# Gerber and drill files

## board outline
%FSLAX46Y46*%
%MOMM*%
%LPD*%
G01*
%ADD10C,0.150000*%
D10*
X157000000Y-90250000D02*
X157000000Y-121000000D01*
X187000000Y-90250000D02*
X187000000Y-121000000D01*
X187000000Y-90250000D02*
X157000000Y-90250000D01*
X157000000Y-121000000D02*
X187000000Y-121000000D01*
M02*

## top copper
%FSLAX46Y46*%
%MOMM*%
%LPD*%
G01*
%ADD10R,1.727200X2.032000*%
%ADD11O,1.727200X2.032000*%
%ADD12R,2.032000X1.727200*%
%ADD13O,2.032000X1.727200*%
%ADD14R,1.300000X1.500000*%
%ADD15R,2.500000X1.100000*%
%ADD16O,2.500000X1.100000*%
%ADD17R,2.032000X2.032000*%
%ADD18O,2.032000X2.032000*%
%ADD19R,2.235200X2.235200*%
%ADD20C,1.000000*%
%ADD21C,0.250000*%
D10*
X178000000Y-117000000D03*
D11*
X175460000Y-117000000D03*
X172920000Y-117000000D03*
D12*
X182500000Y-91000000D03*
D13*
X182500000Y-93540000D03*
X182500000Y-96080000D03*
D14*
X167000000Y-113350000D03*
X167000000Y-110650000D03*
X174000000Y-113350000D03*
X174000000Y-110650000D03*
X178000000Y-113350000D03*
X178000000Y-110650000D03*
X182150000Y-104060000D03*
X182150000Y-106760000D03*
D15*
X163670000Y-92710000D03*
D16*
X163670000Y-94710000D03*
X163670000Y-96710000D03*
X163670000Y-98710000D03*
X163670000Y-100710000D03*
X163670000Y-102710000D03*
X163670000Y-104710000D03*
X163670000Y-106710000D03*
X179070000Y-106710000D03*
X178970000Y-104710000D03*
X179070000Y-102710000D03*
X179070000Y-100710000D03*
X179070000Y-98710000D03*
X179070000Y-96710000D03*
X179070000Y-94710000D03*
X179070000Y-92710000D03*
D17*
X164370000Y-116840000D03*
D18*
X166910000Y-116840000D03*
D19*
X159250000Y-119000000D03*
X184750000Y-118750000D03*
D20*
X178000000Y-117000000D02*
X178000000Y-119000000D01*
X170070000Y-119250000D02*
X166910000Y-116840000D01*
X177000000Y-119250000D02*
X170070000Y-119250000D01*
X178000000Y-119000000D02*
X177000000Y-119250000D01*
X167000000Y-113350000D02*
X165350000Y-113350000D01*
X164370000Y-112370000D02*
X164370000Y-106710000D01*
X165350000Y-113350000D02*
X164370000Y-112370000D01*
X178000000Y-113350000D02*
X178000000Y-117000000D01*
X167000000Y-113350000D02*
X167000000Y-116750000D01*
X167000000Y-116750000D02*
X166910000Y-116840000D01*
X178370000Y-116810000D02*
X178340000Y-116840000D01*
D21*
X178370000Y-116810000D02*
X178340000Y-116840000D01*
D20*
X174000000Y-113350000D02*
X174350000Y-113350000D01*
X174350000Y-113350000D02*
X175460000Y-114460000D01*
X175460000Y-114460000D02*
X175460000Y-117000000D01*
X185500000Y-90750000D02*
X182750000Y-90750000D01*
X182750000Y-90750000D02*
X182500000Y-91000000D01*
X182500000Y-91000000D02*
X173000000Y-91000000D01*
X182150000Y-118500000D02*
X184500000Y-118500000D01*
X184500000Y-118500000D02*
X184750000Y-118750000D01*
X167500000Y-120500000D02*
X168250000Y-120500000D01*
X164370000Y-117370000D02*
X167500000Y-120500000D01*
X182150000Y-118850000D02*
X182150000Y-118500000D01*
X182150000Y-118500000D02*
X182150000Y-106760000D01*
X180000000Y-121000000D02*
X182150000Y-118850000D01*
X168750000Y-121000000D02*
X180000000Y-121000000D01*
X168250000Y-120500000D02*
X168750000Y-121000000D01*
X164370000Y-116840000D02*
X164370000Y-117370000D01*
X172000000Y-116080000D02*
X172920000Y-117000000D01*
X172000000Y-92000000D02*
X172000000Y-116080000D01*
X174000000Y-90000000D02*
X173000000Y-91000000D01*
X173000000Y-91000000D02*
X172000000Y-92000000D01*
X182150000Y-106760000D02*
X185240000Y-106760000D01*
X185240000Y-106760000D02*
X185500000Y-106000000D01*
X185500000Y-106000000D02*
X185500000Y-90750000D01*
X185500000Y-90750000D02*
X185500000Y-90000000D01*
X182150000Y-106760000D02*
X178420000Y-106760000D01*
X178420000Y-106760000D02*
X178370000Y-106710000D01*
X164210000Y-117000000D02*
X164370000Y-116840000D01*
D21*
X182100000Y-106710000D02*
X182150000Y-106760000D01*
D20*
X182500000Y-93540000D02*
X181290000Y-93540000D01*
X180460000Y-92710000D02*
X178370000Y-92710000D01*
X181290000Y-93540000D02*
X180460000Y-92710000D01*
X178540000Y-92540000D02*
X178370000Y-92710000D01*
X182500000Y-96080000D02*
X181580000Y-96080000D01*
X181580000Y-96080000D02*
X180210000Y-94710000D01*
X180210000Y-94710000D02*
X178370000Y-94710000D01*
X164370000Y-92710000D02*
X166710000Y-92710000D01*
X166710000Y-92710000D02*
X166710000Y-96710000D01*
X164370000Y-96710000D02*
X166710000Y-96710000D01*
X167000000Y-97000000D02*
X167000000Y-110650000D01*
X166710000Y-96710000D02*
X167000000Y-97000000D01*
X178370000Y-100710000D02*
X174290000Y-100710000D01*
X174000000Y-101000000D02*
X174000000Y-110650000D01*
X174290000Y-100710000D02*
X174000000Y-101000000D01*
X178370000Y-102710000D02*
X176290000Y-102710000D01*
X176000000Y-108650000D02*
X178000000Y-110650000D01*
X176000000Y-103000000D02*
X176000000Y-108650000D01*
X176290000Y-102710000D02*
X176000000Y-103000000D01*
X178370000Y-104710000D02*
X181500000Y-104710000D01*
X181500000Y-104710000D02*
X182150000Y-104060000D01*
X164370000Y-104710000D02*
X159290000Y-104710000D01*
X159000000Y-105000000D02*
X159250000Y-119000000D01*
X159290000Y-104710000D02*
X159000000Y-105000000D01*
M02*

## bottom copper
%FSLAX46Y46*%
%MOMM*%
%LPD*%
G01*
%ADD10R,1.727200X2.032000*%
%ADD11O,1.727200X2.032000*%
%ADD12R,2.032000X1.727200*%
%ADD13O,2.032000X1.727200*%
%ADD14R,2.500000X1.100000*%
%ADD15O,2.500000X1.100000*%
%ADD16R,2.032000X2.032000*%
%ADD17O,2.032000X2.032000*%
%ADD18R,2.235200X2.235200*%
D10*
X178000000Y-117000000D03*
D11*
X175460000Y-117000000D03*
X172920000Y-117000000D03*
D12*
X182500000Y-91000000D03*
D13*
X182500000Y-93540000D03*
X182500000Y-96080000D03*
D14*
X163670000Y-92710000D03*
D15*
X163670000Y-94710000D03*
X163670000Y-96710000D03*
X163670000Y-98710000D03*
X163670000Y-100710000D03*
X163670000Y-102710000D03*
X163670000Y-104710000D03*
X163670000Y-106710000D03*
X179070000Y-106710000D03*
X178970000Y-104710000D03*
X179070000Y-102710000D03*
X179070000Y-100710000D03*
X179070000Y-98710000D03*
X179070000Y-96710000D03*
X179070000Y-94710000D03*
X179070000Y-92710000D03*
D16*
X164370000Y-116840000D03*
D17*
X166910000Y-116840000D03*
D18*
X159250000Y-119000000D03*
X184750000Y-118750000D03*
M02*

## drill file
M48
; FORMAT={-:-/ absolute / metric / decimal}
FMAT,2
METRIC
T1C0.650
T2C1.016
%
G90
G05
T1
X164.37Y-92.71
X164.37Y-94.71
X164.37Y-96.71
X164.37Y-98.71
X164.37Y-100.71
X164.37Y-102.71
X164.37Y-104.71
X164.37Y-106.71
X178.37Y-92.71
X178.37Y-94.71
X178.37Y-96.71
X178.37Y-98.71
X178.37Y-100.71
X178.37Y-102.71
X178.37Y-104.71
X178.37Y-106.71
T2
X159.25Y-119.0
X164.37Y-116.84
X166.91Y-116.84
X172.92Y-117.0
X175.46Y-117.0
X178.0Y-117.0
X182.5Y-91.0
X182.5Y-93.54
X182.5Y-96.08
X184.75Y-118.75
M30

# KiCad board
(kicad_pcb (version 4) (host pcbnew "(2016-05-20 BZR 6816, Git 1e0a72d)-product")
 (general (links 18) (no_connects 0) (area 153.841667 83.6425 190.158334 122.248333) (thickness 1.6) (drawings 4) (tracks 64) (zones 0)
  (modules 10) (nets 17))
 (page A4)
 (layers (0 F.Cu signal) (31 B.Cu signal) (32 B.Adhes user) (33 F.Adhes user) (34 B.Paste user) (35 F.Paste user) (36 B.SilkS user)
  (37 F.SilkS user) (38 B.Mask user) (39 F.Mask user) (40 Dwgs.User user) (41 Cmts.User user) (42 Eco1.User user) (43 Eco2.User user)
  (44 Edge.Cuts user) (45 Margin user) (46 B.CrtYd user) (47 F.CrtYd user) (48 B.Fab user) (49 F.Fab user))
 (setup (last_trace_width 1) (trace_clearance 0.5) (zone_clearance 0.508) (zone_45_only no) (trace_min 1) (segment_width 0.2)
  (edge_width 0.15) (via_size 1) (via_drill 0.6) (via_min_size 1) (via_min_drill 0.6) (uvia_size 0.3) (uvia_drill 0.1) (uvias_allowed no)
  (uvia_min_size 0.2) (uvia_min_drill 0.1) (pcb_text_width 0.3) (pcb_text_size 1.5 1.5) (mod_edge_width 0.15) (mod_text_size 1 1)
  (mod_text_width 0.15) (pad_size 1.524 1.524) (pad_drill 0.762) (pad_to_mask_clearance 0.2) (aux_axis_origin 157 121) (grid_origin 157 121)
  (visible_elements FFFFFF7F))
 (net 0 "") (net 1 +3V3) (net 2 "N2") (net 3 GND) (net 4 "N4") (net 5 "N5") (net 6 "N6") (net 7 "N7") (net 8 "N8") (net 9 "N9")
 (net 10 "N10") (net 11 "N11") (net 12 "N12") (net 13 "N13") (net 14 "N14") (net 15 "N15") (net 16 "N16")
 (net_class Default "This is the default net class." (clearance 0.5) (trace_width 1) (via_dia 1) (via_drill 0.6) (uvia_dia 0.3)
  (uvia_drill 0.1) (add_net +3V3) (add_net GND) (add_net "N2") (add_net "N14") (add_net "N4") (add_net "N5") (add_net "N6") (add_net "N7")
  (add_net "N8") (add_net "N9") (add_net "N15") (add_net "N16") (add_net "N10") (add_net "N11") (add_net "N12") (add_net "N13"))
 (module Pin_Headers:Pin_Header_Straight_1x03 (layer F.Cu) (at 178 117 270)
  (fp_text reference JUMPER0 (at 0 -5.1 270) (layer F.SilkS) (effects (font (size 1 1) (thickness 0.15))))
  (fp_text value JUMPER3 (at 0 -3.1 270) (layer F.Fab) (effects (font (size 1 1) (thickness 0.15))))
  (pad 1 thru_hole rect (at 0 0 270) (size 2.032 1.7272) (drill 1.016) (layers *.Cu *.Mask F.SilkS) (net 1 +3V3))
  (pad 2 thru_hole oval (at 0 2.54 270) (size 2.032 1.7272) (drill 1.016) (layers *.Cu *.Mask F.SilkS) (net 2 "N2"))
  (pad 3 thru_hole oval (at 0 5.08 270) (size 2.032 1.7272) (drill 1.016) (layers *.Cu *.Mask F.SilkS) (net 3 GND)))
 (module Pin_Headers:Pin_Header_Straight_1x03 (layer F.Cu) (at 182.5 91)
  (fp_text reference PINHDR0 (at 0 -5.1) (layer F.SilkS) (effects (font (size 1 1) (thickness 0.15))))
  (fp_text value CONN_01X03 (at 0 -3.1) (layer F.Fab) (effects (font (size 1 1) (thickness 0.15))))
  (pad 1 thru_hole rect (at 0 0) (size 2.032 1.7272) (drill 1.016) (layers *.Cu *.Mask F.SilkS) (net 3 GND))
  (pad 2 thru_hole oval (at 0 2.54) (size 2.032 1.7272) (drill 1.016) (layers *.Cu *.Mask F.SilkS) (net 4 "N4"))
  (pad 3 thru_hole oval (at 0 5.08) (size 2.032 1.7272) (drill 1.016) (layers *.Cu *.Mask F.SilkS) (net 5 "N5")))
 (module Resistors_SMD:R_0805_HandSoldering (layer F.Cu) (at 167 112 90)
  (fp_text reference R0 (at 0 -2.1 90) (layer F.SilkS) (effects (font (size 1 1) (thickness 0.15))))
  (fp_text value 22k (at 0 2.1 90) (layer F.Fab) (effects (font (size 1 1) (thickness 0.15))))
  (pad 1 smd rect (at -1.35 0 90) (size 1.5 1.3) (layers F.Cu F.Paste F.Mask) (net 1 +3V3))
  (pad 2 smd rect (at 1.35 0 90) (size 1.5 1.3) (layers F.Cu F.Paste F.Mask) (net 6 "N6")))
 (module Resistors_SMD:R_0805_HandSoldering (layer F.Cu) (at 174 112 90)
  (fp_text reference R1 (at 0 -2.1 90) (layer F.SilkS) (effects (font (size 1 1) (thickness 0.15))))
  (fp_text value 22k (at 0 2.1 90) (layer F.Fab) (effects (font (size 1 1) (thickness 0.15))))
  (pad 1 smd rect (at -1.35 0 90) (size 1.5 1.3) (layers F.Cu F.Paste F.Mask) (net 2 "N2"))
  (pad 2 smd rect (at 1.35 0 90) (size 1.5 1.3) (layers F.Cu F.Paste F.Mask) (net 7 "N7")))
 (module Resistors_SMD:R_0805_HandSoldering (layer F.Cu) (at 178 112 90)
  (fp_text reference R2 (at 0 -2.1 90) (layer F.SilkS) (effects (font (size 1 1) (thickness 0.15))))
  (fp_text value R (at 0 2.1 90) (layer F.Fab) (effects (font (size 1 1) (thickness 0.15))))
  (pad 1 smd rect (at -1.35 0 90) (size 1.5 1.3) (layers F.Cu F.Paste F.Mask) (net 1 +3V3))
  (pad 2 smd rect (at 1.35 0 90) (size 1.5 1.3) (layers F.Cu F.Paste F.Mask) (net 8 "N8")))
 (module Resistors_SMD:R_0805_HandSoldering (layer F.Cu) (at 182.15 105.41 270)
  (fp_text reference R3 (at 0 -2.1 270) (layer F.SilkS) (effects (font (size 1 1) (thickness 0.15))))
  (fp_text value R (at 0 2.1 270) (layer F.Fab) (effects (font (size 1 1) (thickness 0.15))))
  (pad 1 smd rect (at -1.35 0 270) (size 1.5 1.3) (layers F.Cu F.Paste F.Mask) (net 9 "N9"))
  (pad 2 smd rect (at 1.35 0 270) (size 1.5 1.3) (layers F.Cu F.Paste F.Mask) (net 3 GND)))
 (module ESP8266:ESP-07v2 (layer F.Cu) (at 164.37 92.71)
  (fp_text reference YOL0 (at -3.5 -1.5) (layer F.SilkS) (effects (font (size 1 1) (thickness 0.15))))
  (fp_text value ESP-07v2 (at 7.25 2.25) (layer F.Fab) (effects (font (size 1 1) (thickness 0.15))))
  (pad 1 thru_hole rect (at 0 0) (size 2.5 1.1) (drill 0.65 (offset -0.7 0)) (layers *.Cu *.Mask F.SilkS) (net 6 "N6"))
  (pad 2 thru_hole oval (at 0 2) (size 2.5 1.1) (drill 0.65 (offset -0.7 0)) (layers *.Cu *.Mask F.SilkS) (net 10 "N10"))
  (pad 3 thru_hole oval (at 0 4) (size 2.5 1.1) (drill 0.65 (offset -0.7 0)) (layers *.Cu *.Mask F.SilkS) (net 6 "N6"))
  (pad 4 thru_hole oval (at 0 6) (size 2.5 1.1) (drill 0.65 (offset -0.7 0)) (layers *.Cu *.Mask F.SilkS) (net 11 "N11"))
  (pad 5 thru_hole oval (at 0 8) (size 2.5 1.1) (drill 0.65 (offset -0.7 0)) (layers *.Cu *.Mask F.SilkS) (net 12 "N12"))
  (pad 6 thru_hole oval (at 0 10) (size 2.5 1.1) (drill 0.65 (offset -0.7 0)) (layers *.Cu *.Mask F.SilkS) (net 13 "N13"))
  (pad 7 thru_hole oval (at 0 12) (size 2.5 1.1) (drill 0.65 (offset -0.7 0)) (layers *.Cu *.Mask F.SilkS) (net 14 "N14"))
  (pad 8 thru_hole oval (at 0 14) (size 2.5 1.1) (drill 0.65 (offset -0.7 0)) (layers *.Cu *.Mask F.SilkS) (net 1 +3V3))
  (pad 9 thru_hole oval (at 14 14) (size 2.5 1.1) (drill 0.65 (offset 0.7 0)) (layers *.Cu *.Mask F.SilkS) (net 3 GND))
  (pad 10 thru_hole oval (at 14 12) (size 2.5 1.1) (drill 0.65 (offset 0.6 0)) (layers *.Cu *.Mask F.SilkS) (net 9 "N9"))
  (pad 11 thru_hole oval (at 14 10) (size 2.5 1.1) (drill 0.65 (offset 0.7 0)) (layers *.Cu *.Mask F.SilkS) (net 8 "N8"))
  (pad 12 thru_hole oval (at 14 8) (size 2.5 1.1) (drill 0.65 (offset 0.7 0)) (layers *.Cu *.Mask F.SilkS) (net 7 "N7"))
  (pad 13 thru_hole oval (at 14 6) (size 2.5 1.1) (drill 0.65 (offset 0.7 0)) (layers *.Cu *.Mask F.SilkS) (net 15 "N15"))
  (pad 14 thru_hole oval (at 14 4) (size 2.5 1.1) (drill 0.65 (offset 0.7 0)) (layers *.Cu *.Mask F.SilkS) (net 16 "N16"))
  (pad 15 thru_hole oval (at 14 2) (size 2.5 1.1) (drill 0.65 (offset 0.7 0)) (layers *.Cu *.Mask F.SilkS) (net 5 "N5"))
  (pad 16 thru_hole oval (at 14 0) (size 2.5 1.1) (drill 0.65 (offset 0.7 0)) (layers *.Cu *.Mask F.SilkS) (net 4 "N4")))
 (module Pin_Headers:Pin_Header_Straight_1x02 (layer F.Cu) (at 164.37 116.84 90)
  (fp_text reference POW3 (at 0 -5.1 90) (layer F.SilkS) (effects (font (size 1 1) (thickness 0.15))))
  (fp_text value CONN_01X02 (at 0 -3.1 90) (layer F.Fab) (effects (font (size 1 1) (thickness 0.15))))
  (pad 1 thru_hole rect (at 0 0 90) (size 2.032 2.032) (drill 1.016) (layers *.Cu *.Mask F.SilkS) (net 3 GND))
  (pad 2 thru_hole oval (at 0 2.54 90) (size 2.032 2.032) (drill 1.016) (layers *.Cu *.Mask F.SilkS) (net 1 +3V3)))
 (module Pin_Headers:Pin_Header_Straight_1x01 (layer F.Cu) (at 159.25 119)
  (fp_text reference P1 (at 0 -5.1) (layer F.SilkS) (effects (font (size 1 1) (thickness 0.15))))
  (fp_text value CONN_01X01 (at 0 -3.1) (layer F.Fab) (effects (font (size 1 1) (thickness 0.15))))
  (pad 1 thru_hole rect (at 0 0) (size 2.2352 2.2352) (drill 1.016) (layers *.Cu *.Mask F.SilkS) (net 14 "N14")))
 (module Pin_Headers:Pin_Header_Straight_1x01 (layer F.Cu) (at 184.75 118.75)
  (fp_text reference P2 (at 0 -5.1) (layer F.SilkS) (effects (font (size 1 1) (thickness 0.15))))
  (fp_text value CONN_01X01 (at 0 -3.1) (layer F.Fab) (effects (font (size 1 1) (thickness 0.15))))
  (pad 1 thru_hole rect (at 0 0) (size 2.2352 2.2352) (drill 1.016) (layers *.Cu *.Mask F.SilkS) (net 3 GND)))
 (gr_line (start 157 90.25) (end 157 121) (angle 90) (layer Edge.Cuts) (width 0.15))
 (gr_line (start 187 90.25) (end 187 121) (angle 90) (layer Edge.Cuts) (width 0.15))
 (gr_line (start 187 90.25) (end 157 90.25) (angle 90) (layer Edge.Cuts) (width 0.15))
 (gr_line (start 157 121) (end 187 121) (angle 90) (layer Edge.Cuts) (width 0.15))
 (segment (start 178 117) (end 178 119) (width 1) (layer F.Cu) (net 1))
 (segment (start 170.07 119.25) (end 166.91 116.84) (width 1) (layer F.Cu) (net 1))
 (segment (start 177 119.25) (end 170.07 119.25) (width 1) (layer F.Cu) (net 1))
 (segment (start 178 119) (end 177 119.25) (width 1) (layer F.Cu) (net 1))
 (segment (start 167 113.35) (end 165.35 113.35) (width 1) (layer F.Cu) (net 1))
 (segment (start 164.37 112.37) (end 164.37 106.71) (width 1) (layer F.Cu) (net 1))
 (segment (start 165.35 113.35) (end 164.37 112.37) (width 1) (layer F.Cu) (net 1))
 (segment (start 178 113.35) (end 178 117) (width 1) (layer F.Cu) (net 1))
 (segment (start 167 113.35) (end 167 116.75) (width 1) (layer F.Cu) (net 1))
 (segment (start 167 116.75) (end 166.91 116.84) (width 1) (layer F.Cu) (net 1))
 (segment (start 178.37 116.81) (end 178.34 116.84) (width 1) (layer F.Cu) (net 1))
 (segment (start 178.37 116.81) (end 178.34 116.84) (width 0.25) (layer F.Cu) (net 1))
 (segment (start 174 113.35) (end 174.35 113.35) (width 1) (layer F.Cu) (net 2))
 (segment (start 174.35 113.35) (end 175.46 114.46) (width 1) (layer F.Cu) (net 2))
 (segment (start 175.46 114.46) (end 175.46 117) (width 1) (layer F.Cu) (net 2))
 (segment (start 185.5 90.75) (end 182.75 90.75) (width 1) (layer F.Cu) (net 3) (status 800000))
 (segment (start 182.75 90.75) (end 182.5 91) (width 1) (layer F.Cu) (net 3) (status C00000))
 (segment (start 182.5 91) (end 173 91) (width 1) (layer F.Cu) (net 3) (status 400000))
 (segment (start 182.15 118.5) (end 184.5 118.5) (width 1) (layer F.Cu) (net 3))
 (segment (start 184.5 118.5) (end 184.75 118.75) (width 1) (layer F.Cu) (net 3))
 (segment (start 167.5 120.5) (end 168.25 120.5) (width 1) (layer F.Cu) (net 3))
 (segment (start 164.37 117.37) (end 167.5 120.5) (width 1) (layer F.Cu) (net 3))
 (segment (start 182.15 118.85) (end 182.15 118.5) (width 1) (layer F.Cu) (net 3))
 (segment (start 182.15 118.5) (end 182.15 106.76) (width 1) (layer F.Cu) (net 3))
 (segment (start 180 121) (end 182.15 118.85) (width 1) (layer F.Cu) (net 3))
 (segment (start 168.75 121) (end 180 121) (width 1) (layer F.Cu) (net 3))
 (segment (start 168.25 120.5) (end 168.75 121) (width 1) (layer F.Cu) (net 3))
 (segment (start 164.37 116.84) (end 164.37 117.37) (width 1) (layer F.Cu) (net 3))
 (segment (start 172 116.08) (end 172.92 117) (width 1) (layer F.Cu) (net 3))
 (segment (start 172 92) (end 172 116.08) (width 1) (layer F.Cu) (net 3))
 (segment (start 174 90) (end 173 91) (width 1) (layer F.Cu) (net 3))
 (segment (start 173 91) (end 172 92) (width 1) (layer F.Cu) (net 3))
 (segment (start 182.15 106.76) (end 185.24 106.76) (width 1) (layer F.Cu) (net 3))
 (segment (start 185.24 106.76) (end 185.5 106) (width 1) (layer F.Cu) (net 3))
 (segment (start 185.5 106) (end 185.5 90.75) (width 1) (layer F.Cu) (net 3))
 (segment (start 185.5 90.75) (end 185.5 90) (width 1) (layer F.Cu) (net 3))
 (segment (start 182.15 106.76) (end 178.42 106.76) (width 1) (layer F.Cu) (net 3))
 (segment (start 178.42 106.76) (end 178.37 106.71) (width 1) (layer F.Cu) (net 3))
 (segment (start 164.21 117) (end 164.37 116.84) (width 1) (layer F.Cu) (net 3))
 (segment (start 182.1 106.71) (end 182.15 106.76) (width 0.25) (layer F.Cu) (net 3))
 (segment (start 182.5 93.54) (end 181.29 93.54) (width 1) (layer F.Cu) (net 4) (status 400000))
 (segment (start 180.46 92.71) (end 178.37 92.71) (width 1) (layer F.Cu) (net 4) (status 800000))
 (segment (start 181.29 93.54) (end 180.46 92.71) (width 1) (layer F.Cu) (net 4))
 (segment (start 178.54 92.54) (end 178.37 92.71) (width 1) (layer F.Cu) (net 4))
 (segment (start 182.5 96.08) (end 181.58 96.08) (width 1) (layer F.Cu) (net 5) (status C00000))
 (segment (start 181.58 96.08) (end 180.21 94.71) (width 1) (layer F.Cu) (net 5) (status C00000))
 (segment (start 180.21 94.71) (end 178.37 94.71) (width 1) (layer F.Cu) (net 5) (status C00000))
 (segment (start 164.37 92.71) (end 166.71 92.71) (width 1) (layer F.Cu) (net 6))
 (segment (start 166.71 92.71) (end 166.71 96.71) (width 1) (layer F.Cu) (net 6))
 (segment (start 164.37 96.71) (end 166.71 96.71) (width 1) (layer F.Cu) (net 6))
 (segment (start 167 97) (end 167 110.65) (width 1) (layer F.Cu) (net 6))
 (segment (start 166.71 96.71) (end 167 97) (width 1) (layer F.Cu) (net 6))
 (segment (start 178.37 100.71) (end 174.29 100.71) (width 1) (layer F.Cu) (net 7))
 (segment (start 174 101) (end 174 110.65) (width 1) (layer F.Cu) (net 7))
 (segment (start 174.29 100.71) (end 174 101) (width 1) (layer F.Cu) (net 7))
 (segment (start 178.37 102.71) (end 176.29 102.71) (width 1) (layer F.Cu) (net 8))
 (segment (start 176 108.65) (end 178 110.65) (width 1) (layer F.Cu) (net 8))
 (segment (start 176 103) (end 176 108.65) (width 1) (layer F.Cu) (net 8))
 (segment (start 176.29 102.71) (end 176 103) (width 1) (layer F.Cu) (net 8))
 (segment (start 178.37 104.71) (end 181.5 104.71) (width 1) (layer F.Cu) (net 9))
 (segment (start 181.5 104.71) (end 182.15 104.06) (width 1) (layer F.Cu) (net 9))
 (segment (start 164.37 104.71) (end 159.29 104.71) (width 1) (layer F.Cu) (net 14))
 (segment (start 159 105) (end 159.25 119) (width 1) (layer F.Cu) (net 14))
 (segment (start 159.29 104.71) (end 159 105) (width 1) (layer F.Cu) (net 14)))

